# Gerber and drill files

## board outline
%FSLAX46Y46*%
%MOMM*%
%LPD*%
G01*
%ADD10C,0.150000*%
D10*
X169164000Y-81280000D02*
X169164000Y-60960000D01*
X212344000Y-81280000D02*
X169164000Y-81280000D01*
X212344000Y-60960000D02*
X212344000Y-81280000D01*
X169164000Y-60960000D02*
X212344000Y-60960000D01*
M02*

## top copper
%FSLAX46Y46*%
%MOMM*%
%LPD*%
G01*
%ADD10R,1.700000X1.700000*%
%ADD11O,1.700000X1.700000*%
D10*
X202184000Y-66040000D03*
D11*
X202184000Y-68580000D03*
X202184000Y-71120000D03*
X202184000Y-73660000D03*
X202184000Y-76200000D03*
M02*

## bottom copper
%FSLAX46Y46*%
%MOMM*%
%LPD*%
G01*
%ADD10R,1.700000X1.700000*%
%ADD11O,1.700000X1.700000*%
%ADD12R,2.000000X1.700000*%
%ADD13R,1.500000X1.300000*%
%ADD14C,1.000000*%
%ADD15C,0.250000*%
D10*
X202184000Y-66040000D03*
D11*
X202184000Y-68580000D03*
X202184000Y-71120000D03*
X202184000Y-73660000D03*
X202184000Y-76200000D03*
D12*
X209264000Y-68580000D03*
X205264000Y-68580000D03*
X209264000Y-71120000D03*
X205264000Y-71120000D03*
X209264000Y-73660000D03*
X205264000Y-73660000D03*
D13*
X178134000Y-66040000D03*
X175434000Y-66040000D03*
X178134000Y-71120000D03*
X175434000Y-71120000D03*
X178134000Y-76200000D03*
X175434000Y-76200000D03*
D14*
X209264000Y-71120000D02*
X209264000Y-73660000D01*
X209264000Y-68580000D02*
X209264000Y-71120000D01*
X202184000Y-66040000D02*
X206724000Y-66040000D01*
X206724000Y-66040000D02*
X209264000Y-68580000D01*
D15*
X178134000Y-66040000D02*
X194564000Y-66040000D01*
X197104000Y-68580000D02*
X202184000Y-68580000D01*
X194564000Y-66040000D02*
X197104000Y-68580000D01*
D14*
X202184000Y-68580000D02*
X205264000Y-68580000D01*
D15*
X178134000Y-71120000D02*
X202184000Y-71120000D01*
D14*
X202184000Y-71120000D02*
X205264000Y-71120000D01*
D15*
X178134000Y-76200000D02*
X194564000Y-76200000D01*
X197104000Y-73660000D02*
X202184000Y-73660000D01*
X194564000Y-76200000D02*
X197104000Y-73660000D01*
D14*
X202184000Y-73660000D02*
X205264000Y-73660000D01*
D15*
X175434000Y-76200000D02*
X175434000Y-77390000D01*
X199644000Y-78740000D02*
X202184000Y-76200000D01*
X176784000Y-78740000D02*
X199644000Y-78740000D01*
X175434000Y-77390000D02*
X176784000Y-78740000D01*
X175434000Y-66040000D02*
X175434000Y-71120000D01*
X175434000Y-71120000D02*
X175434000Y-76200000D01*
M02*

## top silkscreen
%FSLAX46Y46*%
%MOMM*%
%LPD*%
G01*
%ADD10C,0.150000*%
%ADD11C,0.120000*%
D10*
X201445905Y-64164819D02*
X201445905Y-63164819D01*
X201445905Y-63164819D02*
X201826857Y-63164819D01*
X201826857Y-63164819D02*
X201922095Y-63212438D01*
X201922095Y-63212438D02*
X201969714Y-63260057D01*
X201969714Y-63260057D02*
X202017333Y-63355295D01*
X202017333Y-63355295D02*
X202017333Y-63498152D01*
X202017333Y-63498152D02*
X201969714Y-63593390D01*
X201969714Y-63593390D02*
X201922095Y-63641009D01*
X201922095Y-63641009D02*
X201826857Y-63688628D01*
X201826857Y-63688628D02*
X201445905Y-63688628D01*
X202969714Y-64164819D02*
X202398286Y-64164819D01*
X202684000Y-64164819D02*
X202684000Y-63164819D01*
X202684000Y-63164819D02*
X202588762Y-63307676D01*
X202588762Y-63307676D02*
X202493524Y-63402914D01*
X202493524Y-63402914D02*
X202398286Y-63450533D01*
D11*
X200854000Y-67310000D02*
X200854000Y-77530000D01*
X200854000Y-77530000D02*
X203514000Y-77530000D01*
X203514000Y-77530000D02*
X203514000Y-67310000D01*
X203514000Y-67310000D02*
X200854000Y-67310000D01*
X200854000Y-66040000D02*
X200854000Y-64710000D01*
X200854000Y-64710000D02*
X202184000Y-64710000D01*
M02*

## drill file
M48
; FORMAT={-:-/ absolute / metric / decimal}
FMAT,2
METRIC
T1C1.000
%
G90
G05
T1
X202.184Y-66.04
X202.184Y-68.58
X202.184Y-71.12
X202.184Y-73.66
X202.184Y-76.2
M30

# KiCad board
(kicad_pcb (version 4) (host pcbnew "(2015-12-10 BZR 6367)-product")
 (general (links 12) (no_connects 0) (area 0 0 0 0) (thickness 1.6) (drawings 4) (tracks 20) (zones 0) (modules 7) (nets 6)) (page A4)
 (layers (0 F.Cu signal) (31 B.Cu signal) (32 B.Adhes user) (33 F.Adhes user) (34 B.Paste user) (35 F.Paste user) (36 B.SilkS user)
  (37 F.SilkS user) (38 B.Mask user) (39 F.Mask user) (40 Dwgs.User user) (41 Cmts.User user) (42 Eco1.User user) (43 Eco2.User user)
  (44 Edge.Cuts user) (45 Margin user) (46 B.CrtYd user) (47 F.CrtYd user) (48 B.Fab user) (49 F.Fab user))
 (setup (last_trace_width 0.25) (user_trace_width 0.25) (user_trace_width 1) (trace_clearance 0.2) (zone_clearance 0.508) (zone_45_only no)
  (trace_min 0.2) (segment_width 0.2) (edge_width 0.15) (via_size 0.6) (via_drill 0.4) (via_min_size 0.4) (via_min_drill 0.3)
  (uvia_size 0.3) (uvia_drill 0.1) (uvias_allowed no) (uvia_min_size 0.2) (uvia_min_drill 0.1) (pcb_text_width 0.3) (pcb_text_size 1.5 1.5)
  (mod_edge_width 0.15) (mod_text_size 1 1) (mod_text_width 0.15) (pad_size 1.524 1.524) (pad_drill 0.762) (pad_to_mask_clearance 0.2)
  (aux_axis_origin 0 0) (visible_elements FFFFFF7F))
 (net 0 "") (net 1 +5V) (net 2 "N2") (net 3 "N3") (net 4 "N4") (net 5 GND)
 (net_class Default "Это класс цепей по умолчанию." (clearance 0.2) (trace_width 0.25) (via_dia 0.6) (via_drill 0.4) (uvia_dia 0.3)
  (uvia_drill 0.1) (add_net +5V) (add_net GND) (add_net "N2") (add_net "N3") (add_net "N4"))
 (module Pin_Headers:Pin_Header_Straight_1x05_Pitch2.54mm (layer F.Cu) (at 202.184 66.04)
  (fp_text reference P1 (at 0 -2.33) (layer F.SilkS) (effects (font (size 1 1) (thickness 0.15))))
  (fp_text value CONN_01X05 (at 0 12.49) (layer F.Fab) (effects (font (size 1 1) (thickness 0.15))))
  (fp_line (start -1.33 1.27) (end -1.33 11.49) (layer F.SilkS) (width 0.12))
  (fp_line (start -1.33 11.49) (end 1.33 11.49) (layer F.SilkS) (width 0.12))
  (fp_line (start 1.33 11.49) (end 1.33 1.27) (layer F.SilkS) (width 0.12))
  (fp_line (start 1.33 1.27) (end -1.33 1.27) (layer F.SilkS) (width 0.12))
  (fp_line (start -1.33 0) (end -1.33 -1.33) (layer F.SilkS) (width 0.12))
  (fp_line (start -1.33 -1.33) (end 0 -1.33) (layer F.SilkS) (width 0.12))
  (pad 1 thru_hole rect (at 0 0) (size 1.7 1.7) (drill 1) (layers *.Cu *.Mask) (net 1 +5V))
  (pad 2 thru_hole oval (at 0 2.54) (size 1.7 1.7) (drill 1) (layers *.Cu *.Mask) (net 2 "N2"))
  (pad 3 thru_hole oval (at 0 5.08) (size 1.7 1.7) (drill 1) (layers *.Cu *.Mask) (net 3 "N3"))
  (pad 4 thru_hole oval (at 0 7.62) (size 1.7 1.7) (drill 1) (layers *.Cu *.Mask) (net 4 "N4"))
  (pad 5 thru_hole oval (at 0 10.16) (size 1.7 1.7) (drill 1) (layers *.Cu *.Mask) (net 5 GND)))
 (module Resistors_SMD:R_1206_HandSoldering (layer B.Cu) (at 207.264 68.58 180)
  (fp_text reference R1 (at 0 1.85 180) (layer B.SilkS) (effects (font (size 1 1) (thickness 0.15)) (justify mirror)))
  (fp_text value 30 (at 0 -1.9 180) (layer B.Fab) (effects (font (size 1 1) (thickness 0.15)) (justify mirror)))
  (pad 1 smd rect (at -2 0 180) (size 2 1.7) (layers B.Cu B.Paste B.Mask) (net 1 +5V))
  (pad 2 smd rect (at 2 0 180) (size 2 1.7) (layers B.Cu B.Paste B.Mask) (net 2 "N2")))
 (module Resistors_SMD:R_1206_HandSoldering (layer B.Cu) (at 207.264 71.12 180)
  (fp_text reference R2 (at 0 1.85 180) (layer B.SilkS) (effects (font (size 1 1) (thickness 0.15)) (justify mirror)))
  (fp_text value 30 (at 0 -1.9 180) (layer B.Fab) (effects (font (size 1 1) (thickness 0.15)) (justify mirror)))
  (pad 1 smd rect (at -2 0 180) (size 2 1.7) (layers B.Cu B.Paste B.Mask) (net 1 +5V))
  (pad 2 smd rect (at 2 0 180) (size 2 1.7) (layers B.Cu B.Paste B.Mask) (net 3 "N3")))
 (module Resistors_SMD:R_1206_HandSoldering (layer B.Cu) (at 207.264 73.66 180)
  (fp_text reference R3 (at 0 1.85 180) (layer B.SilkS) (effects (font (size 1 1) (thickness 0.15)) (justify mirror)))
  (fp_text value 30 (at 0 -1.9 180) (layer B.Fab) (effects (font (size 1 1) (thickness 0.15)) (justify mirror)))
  (pad 1 smd rect (at -2 0 180) (size 2 1.7) (layers B.Cu B.Paste B.Mask) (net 1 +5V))
  (pad 2 smd rect (at 2 0 180) (size 2 1.7) (layers B.Cu B.Paste B.Mask) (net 4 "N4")))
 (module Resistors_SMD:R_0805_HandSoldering (layer B.Cu) (at 176.784 66.04 180)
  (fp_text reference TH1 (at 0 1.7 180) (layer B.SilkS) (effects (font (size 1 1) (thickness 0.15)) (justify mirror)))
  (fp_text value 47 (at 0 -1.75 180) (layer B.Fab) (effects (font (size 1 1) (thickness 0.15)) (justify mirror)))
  (pad 1 smd rect (at -1.35 0 180) (size 1.5 1.3) (layers B.Cu B.Paste B.Mask) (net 2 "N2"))
  (pad 2 smd rect (at 1.35 0 180) (size 1.5 1.3) (layers B.Cu B.Paste B.Mask) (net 5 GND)))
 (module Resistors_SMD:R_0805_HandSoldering (layer B.Cu) (at 176.784 71.12 180)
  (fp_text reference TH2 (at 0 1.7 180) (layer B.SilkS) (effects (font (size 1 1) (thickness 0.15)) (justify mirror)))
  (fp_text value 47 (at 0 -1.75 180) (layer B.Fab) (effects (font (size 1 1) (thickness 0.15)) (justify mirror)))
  (pad 1 smd rect (at -1.35 0 180) (size 1.5 1.3) (layers B.Cu B.Paste B.Mask) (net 3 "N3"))
  (pad 2 smd rect (at 1.35 0 180) (size 1.5 1.3) (layers B.Cu B.Paste B.Mask) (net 5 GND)))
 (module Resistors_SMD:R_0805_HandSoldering (layer B.Cu) (at 176.784 76.2 180)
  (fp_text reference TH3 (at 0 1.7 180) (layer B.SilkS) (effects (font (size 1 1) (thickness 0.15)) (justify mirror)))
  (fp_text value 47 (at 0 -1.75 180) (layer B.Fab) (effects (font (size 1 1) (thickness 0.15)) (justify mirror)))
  (pad 1 smd rect (at -1.35 0 180) (size 1.5 1.3) (layers B.Cu B.Paste B.Mask) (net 4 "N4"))
  (pad 2 smd rect (at 1.35 0 180) (size 1.5 1.3) (layers B.Cu B.Paste B.Mask) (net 5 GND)))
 (gr_line (start 169.164 81.28) (end 169.164 60.96) (angle 90) (layer Edge.Cuts) (width 0.15))
 (gr_line (start 212.344 81.28) (end 169.164 81.28) (angle 90) (layer Edge.Cuts) (width 0.15))
 (gr_line (start 212.344 60.96) (end 212.344 81.28) (angle 90) (layer Edge.Cuts) (width 0.15))
 (gr_line (start 169.164 60.96) (end 212.344 60.96) (angle 90) (layer Edge.Cuts) (width 0.15))
 (segment (start 209.264 71.12) (end 209.264 73.66) (width 1) (layer B.Cu) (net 1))
 (segment (start 209.264 68.58) (end 209.264 71.12) (width 1) (layer B.Cu) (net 1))
 (segment (start 202.184 66.04) (end 206.724 66.04) (width 1) (layer B.Cu) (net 1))
 (segment (start 206.724 66.04) (end 209.264 68.58) (width 1) (layer B.Cu) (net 1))
 (segment (start 178.134 66.04) (end 194.564 66.04) (width 0.25) (layer B.Cu) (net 2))
 (segment (start 197.104 68.58) (end 202.184 68.58) (width 0.25) (layer B.Cu) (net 2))
 (segment (start 194.564 66.04) (end 197.104 68.58) (width 0.25) (layer B.Cu) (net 2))
 (segment (start 202.184 68.58) (end 205.264 68.58) (width 1) (layer B.Cu) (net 2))
 (segment (start 178.134 71.12) (end 202.184 71.12) (width 0.25) (layer B.Cu) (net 3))
 (segment (start 202.184 71.12) (end 205.264 71.12) (width 1) (layer B.Cu) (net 3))
 (segment (start 178.134 76.2) (end 194.564 76.2) (width 0.25) (layer B.Cu) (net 4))
 (segment (start 197.104 73.66) (end 202.184 73.66) (width 0.25) (layer B.Cu) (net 4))
 (segment (start 194.564 76.2) (end 197.104 73.66) (width 0.25) (layer B.Cu) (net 4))
 (segment (start 202.184 73.66) (end 205.264 73.66) (width 1) (layer B.Cu) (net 4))
 (segment (start 175.434 76.2) (end 175.434 77.39) (width 0.25) (layer B.Cu) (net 5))
 (segment (start 199.644 78.74) (end 202.184 76.2) (width 0.25) (layer B.Cu) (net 5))
 (segment (start 176.784 78.74) (end 199.644 78.74) (width 0.25) (layer B.Cu) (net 5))
 (segment (start 175.434 77.39) (end 176.784 78.74) (width 0.25) (layer B.Cu) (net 5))
 (segment (start 175.434 66.04) (end 175.434 71.12) (width 0.25) (layer B.Cu) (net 5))
 (segment (start 175.434 71.12) (end 175.434 76.2) (width 0.25) (layer B.Cu) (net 5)))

